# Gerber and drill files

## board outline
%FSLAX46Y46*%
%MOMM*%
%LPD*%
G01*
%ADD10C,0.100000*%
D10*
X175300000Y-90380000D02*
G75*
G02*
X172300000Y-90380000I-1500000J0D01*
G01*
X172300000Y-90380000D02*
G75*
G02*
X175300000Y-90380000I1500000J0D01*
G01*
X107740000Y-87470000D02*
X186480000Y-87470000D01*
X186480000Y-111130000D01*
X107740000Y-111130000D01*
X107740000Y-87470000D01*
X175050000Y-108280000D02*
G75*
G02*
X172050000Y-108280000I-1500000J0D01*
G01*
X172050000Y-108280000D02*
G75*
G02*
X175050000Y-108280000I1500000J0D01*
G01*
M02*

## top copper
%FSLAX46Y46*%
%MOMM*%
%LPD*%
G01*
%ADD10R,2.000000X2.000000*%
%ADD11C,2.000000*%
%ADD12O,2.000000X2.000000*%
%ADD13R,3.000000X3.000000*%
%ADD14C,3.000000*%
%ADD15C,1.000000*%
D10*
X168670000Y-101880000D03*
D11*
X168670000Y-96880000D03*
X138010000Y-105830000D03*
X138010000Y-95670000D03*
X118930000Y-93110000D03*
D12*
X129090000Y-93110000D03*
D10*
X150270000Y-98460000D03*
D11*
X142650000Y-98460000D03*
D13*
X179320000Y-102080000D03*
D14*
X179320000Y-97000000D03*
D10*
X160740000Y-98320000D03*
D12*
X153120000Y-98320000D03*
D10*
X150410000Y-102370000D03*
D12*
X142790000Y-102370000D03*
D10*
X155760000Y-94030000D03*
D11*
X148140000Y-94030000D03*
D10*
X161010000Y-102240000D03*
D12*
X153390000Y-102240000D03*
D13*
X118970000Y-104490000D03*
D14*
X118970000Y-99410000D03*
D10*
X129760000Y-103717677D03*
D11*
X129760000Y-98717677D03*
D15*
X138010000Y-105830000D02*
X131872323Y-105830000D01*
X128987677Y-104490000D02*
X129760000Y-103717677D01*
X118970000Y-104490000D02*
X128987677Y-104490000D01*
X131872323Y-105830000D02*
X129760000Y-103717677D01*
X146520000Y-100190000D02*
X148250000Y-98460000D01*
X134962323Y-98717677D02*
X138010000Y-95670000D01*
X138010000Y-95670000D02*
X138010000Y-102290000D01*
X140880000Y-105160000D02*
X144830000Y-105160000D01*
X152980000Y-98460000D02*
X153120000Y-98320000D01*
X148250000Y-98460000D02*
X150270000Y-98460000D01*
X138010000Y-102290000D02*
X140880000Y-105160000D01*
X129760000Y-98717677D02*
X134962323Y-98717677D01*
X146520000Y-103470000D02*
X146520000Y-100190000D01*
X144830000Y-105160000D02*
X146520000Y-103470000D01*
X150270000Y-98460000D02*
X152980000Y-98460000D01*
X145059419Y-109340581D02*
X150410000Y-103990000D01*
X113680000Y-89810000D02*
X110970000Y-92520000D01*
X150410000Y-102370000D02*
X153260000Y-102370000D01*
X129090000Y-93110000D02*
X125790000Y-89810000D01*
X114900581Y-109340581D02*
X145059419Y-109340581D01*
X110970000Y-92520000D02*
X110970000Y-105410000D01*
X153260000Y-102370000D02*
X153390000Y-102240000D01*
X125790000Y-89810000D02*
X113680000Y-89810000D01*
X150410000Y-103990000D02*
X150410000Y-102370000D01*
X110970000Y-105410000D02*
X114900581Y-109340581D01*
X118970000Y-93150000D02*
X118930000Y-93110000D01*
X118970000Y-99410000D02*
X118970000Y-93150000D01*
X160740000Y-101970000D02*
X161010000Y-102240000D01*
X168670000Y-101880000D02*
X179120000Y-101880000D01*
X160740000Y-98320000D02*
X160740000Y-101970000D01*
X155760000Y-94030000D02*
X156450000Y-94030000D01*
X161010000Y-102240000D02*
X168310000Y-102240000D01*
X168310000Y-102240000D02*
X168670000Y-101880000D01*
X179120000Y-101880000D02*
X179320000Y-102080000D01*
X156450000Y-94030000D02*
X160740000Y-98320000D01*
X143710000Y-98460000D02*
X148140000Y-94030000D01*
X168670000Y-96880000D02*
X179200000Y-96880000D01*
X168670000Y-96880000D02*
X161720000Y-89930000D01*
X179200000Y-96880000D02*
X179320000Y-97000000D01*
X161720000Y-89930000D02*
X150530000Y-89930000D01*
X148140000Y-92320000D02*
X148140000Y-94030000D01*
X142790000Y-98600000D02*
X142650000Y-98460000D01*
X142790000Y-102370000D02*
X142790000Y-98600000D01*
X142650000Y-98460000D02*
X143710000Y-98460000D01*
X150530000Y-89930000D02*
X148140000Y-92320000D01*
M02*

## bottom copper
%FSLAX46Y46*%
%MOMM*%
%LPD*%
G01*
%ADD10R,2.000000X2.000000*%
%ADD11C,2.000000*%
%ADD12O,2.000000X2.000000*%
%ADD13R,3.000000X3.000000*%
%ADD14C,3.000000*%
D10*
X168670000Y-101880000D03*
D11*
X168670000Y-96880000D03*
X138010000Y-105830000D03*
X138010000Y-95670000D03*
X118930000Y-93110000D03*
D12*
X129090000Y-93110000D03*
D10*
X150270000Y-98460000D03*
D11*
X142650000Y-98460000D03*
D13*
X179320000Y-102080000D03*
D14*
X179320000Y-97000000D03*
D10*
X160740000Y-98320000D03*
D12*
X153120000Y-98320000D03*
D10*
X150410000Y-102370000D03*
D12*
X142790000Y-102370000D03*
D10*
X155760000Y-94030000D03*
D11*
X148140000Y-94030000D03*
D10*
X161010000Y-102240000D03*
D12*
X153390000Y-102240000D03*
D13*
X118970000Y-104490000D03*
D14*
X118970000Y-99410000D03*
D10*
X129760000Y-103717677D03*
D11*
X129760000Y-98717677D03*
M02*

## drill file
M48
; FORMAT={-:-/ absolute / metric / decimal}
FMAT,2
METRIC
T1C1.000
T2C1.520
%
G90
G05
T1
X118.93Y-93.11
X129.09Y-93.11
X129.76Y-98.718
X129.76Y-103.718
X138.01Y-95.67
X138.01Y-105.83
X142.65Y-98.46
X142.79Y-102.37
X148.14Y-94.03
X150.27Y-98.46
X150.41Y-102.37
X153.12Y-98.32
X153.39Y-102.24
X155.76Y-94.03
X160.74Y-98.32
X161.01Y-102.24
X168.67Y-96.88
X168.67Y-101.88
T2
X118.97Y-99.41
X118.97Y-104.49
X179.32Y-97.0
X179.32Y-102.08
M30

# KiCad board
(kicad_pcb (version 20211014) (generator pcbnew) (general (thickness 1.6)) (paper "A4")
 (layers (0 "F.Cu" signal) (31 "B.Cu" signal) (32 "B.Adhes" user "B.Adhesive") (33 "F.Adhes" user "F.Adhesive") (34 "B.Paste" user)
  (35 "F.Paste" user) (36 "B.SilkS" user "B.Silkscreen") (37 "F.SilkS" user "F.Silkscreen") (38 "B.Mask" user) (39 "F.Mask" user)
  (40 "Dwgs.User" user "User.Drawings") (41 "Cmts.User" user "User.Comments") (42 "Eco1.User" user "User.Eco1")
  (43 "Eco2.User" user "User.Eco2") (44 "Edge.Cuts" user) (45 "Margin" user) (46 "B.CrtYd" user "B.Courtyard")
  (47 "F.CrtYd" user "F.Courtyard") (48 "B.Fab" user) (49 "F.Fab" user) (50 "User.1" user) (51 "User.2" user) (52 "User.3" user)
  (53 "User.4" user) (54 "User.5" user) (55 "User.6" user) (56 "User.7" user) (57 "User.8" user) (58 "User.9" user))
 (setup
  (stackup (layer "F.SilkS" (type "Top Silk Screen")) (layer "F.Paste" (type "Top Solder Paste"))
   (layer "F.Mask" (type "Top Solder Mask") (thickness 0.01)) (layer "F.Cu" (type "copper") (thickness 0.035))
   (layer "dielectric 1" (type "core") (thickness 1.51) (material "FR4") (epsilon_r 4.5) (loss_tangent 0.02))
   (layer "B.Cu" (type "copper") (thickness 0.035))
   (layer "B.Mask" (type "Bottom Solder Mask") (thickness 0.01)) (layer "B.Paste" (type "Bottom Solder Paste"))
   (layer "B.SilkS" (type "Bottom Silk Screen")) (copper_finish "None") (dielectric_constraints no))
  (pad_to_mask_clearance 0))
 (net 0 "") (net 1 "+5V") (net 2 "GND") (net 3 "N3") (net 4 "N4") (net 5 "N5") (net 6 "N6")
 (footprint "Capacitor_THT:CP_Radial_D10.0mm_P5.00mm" (layer "F.Cu") (at 168.67 101.88 90)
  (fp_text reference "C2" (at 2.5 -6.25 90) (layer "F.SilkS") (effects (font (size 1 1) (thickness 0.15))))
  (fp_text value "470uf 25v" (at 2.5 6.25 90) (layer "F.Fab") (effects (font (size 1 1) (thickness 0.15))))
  (pad "1" thru_hole rect (at 0 0 90) (size 2 2) (drill 1) (layers *.Cu *.Mask) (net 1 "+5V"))
  (pad "2" thru_hole circle (at 5 0 90) (size 2 2) (drill 1) (layers *.Cu *.Mask) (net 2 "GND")))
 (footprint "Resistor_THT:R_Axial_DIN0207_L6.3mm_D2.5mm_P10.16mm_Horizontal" (layer "F.Cu") (at 138.01 105.83 90)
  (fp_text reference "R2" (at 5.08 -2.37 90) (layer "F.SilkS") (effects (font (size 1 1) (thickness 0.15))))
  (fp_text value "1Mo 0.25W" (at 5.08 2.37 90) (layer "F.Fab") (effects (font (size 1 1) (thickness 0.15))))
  (pad "1" thru_hole circle (at 0 0 90) (size 2 2) (drill 1) (layers *.Cu *.Mask) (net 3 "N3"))
  (pad "2" thru_hole circle (at 10.16 0 90) (size 2 2) (drill 1) (layers *.Cu *.Mask) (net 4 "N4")))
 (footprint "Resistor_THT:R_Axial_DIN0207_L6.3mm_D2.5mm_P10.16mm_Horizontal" (layer "F.Cu") (at 118.93 93.11)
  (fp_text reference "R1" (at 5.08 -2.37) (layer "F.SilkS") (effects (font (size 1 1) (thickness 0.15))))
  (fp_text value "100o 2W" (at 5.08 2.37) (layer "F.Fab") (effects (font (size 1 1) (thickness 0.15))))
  (pad "1" thru_hole circle (at 0 0) (size 2 2) (drill 1) (layers *.Cu *.Mask) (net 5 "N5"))
  (pad "2" thru_hole oval (at 10.16 0) (size 2 2) (drill 1) (layers *.Cu *.Mask) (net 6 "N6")))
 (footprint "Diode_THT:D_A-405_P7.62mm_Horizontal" (layer "F.Cu") (at 150.27 98.46 180)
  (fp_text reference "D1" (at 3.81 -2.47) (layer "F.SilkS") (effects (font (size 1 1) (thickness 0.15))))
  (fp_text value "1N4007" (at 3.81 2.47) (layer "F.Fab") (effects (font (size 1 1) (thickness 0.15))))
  (pad "1" thru_hole rect (at 0 0 180) (size 2 2) (drill 1) (layers *.Cu *.Mask) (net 4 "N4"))
  (pad "2" thru_hole circle (at 7.62 0 180) (size 2 2) (drill 1) (layers *.Cu *.Mask) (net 2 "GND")))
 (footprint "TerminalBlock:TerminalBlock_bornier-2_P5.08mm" (layer "F.Cu") (at 179.32 102.08 90)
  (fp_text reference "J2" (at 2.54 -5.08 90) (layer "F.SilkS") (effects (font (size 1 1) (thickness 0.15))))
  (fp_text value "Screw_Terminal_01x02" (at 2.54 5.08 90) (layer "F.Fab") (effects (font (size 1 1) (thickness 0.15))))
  (pad "1" thru_hole rect (at 0 0 90) (size 3 3) (drill 1.52) (layers *.Cu *.Mask) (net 1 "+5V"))
  (pad "2" thru_hole circle (at 5.08 0 90) (size 3 3) (drill 1.52) (layers *.Cu *.Mask) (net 2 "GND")))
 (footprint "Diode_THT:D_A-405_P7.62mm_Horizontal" (layer "F.Cu") (at 160.74 98.32 180)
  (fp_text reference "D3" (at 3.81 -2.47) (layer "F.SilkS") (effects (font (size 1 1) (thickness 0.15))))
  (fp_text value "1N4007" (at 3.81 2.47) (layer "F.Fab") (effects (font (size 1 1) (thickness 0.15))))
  (pad "1" thru_hole rect (at 0 0 180) (size 2 2) (drill 1) (layers *.Cu *.Mask) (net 1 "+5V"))
  (pad "2" thru_hole oval (at 7.62 0 180) (size 2 2) (drill 1) (layers *.Cu *.Mask) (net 4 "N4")))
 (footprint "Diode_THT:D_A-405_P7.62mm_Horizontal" (layer "F.Cu") (at 150.41 102.37 180)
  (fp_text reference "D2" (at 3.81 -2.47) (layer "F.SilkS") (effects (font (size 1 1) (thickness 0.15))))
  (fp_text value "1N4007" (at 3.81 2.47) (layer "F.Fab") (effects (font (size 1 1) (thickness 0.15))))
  (pad "1" thru_hole rect (at 0 0 180) (size 2 2) (drill 1) (layers *.Cu *.Mask) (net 6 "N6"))
  (pad "2" thru_hole oval (at 7.62 0 180) (size 2 2) (drill 1) (layers *.Cu *.Mask) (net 2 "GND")))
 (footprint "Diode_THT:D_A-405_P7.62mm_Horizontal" (layer "F.Cu") (at 155.76 94.03 180)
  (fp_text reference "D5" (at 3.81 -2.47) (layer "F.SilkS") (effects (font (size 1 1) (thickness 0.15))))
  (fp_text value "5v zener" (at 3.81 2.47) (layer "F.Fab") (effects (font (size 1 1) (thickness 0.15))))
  (pad "1" thru_hole rect (at 0 0 180) (size 2 2) (drill 1) (layers *.Cu *.Mask) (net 1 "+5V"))
  (pad "2" thru_hole circle (at 7.62 0 180) (size 2 2) (drill 1) (layers *.Cu *.Mask) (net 2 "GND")))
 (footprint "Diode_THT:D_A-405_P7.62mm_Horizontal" (layer "F.Cu") (at 161.01 102.24 180)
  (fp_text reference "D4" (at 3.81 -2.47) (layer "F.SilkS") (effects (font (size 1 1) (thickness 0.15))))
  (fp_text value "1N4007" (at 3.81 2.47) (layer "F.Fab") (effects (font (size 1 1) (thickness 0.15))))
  (pad "1" thru_hole rect (at 0 0 180) (size 2 2) (drill 1) (layers *.Cu *.Mask) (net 1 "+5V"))
  (pad "2" thru_hole oval (at 7.62 0 180) (size 2 2) (drill 1) (layers *.Cu *.Mask) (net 6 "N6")))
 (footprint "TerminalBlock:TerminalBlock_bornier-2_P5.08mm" (layer "F.Cu") (at 118.97 104.49 90)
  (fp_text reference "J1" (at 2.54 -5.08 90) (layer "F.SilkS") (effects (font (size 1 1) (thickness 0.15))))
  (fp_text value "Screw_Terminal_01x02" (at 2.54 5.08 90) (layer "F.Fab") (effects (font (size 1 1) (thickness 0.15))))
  (pad "1" thru_hole rect (at 0 0 90) (size 3 3) (drill 1.52) (layers *.Cu *.Mask) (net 3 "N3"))
  (pad "2" thru_hole circle (at 5.08 0 90) (size 3 3) (drill 1.52) (layers *.Cu *.Mask) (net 5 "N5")))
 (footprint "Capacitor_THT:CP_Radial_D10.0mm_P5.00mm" (layer "F.Cu") (at 129.76 103.717677 90)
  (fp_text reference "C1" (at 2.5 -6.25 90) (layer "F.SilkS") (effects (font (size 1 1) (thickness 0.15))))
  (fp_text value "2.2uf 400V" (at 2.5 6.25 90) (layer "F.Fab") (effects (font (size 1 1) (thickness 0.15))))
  (pad "1" thru_hole rect (at 0 0 90) (size 2 2) (drill 1) (layers *.Cu *.Mask) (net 3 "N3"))
  (pad "2" thru_hole circle (at 5 0 90) (size 2 2) (drill 1) (layers *.Cu *.Mask) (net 4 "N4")))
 (gr_circle (center 173.8 90.38) (end 175.3 90.38) (layer "Edge.Cuts") (width 0.1) (fill none))
 (gr_rect (start 107.74 87.47) (end 186.48 111.13) (layer "Edge.Cuts") (width 0.1) (fill none))
 (gr_circle (center 173.55 108.28) (end 175.05 108.28) (layer "Edge.Cuts") (width 0.1) (fill none))
 (segment (start 138.01 105.83) (end 131.872323 105.83) (width 1) (layer "F.Cu") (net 3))
 (segment (start 128.987677 104.49) (end 129.76 103.717677) (width 1) (layer "F.Cu") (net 3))
 (segment (start 118.97 104.49) (end 128.987677 104.49) (width 1) (layer "F.Cu") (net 3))
 (segment (start 131.872323 105.83) (end 129.76 103.717677) (width 1) (layer "F.Cu") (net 3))
 (segment (start 146.52 100.19) (end 148.25 98.46) (width 1) (layer "F.Cu") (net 4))
 (segment (start 134.962323 98.717677) (end 138.01 95.67) (width 1) (layer "F.Cu") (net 4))
 (segment (start 138.01 95.67) (end 138.01 102.29) (width 1) (layer "F.Cu") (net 4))
 (segment (start 140.88 105.16) (end 144.83 105.16) (width 1) (layer "F.Cu") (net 4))
 (segment (start 152.98 98.46) (end 153.12 98.32) (width 1) (layer "F.Cu") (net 4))
 (segment (start 148.25 98.46) (end 150.27 98.46) (width 1) (layer "F.Cu") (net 4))
 (segment (start 138.01 102.29) (end 140.88 105.16) (width 1) (layer "F.Cu") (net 4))
 (segment (start 129.76 98.717677) (end 134.962323 98.717677) (width 1) (layer "F.Cu") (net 4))
 (segment (start 146.52 103.47) (end 146.52 100.19) (width 1) (layer "F.Cu") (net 4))
 (segment (start 144.83 105.16) (end 146.52 103.47) (width 1) (layer "F.Cu") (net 4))
 (segment (start 150.27 98.46) (end 152.98 98.46) (width 1) (layer "F.Cu") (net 4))
 (segment (start 145.059419 109.340581) (end 150.41 103.99) (width 1) (layer "F.Cu") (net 6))
 (segment (start 113.68 89.81) (end 110.97 92.52) (width 1) (layer "F.Cu") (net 6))
 (segment (start 150.41 102.37) (end 153.26 102.37) (width 1) (layer "F.Cu") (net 6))
 (segment (start 129.09 93.11) (end 125.79 89.81) (width 1) (layer "F.Cu") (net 6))
 (segment (start 114.900581 109.340581) (end 145.059419 109.340581) (width 1) (layer "F.Cu") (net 6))
 (segment (start 110.97 92.52) (end 110.97 105.41) (width 1) (layer "F.Cu") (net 6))
 (segment (start 153.26 102.37) (end 153.39 102.24) (width 1) (layer "F.Cu") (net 6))
 (segment (start 125.79 89.81) (end 113.68 89.81) (width 1) (layer "F.Cu") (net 6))
 (segment (start 150.41 103.99) (end 150.41 102.37) (width 1) (layer "F.Cu") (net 6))
 (segment (start 110.97 105.41) (end 114.900581 109.340581) (width 1) (layer "F.Cu") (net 6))
 (segment (start 118.97 93.15) (end 118.93 93.11) (width 1) (layer "F.Cu") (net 5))
 (segment (start 118.97 99.41) (end 118.97 93.15) (width 1) (layer "F.Cu") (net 5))
 (segment (start 160.74 101.97) (end 161.01 102.24) (width 1) (layer "F.Cu") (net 1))
 (segment (start 168.67 101.88) (end 179.12 101.88) (width 1) (layer "F.Cu") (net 1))
 (segment (start 160.74 98.32) (end 160.74 101.97) (width 1) (layer "F.Cu") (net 1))
 (segment (start 155.76 94.03) (end 156.45 94.03) (width 1) (layer "F.Cu") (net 1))
 (segment (start 161.01 102.24) (end 168.31 102.24) (width 1) (layer "F.Cu") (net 1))
 (segment (start 168.31 102.24) (end 168.67 101.88) (width 1) (layer "F.Cu") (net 1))
 (segment (start 179.12 101.88) (end 179.32 102.08) (width 1) (layer "F.Cu") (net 1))
 (segment (start 156.45 94.03) (end 160.74 98.32) (width 1) (layer "F.Cu") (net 1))
 (segment (start 143.71 98.46) (end 148.14 94.03) (width 1) (layer "F.Cu") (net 2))
 (segment (start 168.67 96.88) (end 179.2 96.88) (width 1) (layer "F.Cu") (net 2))
 (segment (start 168.67 96.88) (end 161.72 89.93) (width 1) (layer "F.Cu") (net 2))
 (segment (start 179.2 96.88) (end 179.32 97) (width 1) (layer "F.Cu") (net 2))
 (segment (start 161.72 89.93) (end 150.53 89.93) (width 1) (layer "F.Cu") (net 2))
 (segment (start 148.14 92.32) (end 148.14 94.03) (width 1) (layer "F.Cu") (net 2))
 (segment (start 142.79 98.6) (end 142.65 98.46) (width 1) (layer "F.Cu") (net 2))
 (segment (start 142.79 102.37) (end 142.79 98.6) (width 1) (layer "F.Cu") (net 2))
 (segment (start 142.65 98.46) (end 143.71 98.46) (width 1) (layer "F.Cu") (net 2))
 (segment (start 150.53 89.93) (end 148.14 92.32) (width 1) (layer "F.Cu") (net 2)))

